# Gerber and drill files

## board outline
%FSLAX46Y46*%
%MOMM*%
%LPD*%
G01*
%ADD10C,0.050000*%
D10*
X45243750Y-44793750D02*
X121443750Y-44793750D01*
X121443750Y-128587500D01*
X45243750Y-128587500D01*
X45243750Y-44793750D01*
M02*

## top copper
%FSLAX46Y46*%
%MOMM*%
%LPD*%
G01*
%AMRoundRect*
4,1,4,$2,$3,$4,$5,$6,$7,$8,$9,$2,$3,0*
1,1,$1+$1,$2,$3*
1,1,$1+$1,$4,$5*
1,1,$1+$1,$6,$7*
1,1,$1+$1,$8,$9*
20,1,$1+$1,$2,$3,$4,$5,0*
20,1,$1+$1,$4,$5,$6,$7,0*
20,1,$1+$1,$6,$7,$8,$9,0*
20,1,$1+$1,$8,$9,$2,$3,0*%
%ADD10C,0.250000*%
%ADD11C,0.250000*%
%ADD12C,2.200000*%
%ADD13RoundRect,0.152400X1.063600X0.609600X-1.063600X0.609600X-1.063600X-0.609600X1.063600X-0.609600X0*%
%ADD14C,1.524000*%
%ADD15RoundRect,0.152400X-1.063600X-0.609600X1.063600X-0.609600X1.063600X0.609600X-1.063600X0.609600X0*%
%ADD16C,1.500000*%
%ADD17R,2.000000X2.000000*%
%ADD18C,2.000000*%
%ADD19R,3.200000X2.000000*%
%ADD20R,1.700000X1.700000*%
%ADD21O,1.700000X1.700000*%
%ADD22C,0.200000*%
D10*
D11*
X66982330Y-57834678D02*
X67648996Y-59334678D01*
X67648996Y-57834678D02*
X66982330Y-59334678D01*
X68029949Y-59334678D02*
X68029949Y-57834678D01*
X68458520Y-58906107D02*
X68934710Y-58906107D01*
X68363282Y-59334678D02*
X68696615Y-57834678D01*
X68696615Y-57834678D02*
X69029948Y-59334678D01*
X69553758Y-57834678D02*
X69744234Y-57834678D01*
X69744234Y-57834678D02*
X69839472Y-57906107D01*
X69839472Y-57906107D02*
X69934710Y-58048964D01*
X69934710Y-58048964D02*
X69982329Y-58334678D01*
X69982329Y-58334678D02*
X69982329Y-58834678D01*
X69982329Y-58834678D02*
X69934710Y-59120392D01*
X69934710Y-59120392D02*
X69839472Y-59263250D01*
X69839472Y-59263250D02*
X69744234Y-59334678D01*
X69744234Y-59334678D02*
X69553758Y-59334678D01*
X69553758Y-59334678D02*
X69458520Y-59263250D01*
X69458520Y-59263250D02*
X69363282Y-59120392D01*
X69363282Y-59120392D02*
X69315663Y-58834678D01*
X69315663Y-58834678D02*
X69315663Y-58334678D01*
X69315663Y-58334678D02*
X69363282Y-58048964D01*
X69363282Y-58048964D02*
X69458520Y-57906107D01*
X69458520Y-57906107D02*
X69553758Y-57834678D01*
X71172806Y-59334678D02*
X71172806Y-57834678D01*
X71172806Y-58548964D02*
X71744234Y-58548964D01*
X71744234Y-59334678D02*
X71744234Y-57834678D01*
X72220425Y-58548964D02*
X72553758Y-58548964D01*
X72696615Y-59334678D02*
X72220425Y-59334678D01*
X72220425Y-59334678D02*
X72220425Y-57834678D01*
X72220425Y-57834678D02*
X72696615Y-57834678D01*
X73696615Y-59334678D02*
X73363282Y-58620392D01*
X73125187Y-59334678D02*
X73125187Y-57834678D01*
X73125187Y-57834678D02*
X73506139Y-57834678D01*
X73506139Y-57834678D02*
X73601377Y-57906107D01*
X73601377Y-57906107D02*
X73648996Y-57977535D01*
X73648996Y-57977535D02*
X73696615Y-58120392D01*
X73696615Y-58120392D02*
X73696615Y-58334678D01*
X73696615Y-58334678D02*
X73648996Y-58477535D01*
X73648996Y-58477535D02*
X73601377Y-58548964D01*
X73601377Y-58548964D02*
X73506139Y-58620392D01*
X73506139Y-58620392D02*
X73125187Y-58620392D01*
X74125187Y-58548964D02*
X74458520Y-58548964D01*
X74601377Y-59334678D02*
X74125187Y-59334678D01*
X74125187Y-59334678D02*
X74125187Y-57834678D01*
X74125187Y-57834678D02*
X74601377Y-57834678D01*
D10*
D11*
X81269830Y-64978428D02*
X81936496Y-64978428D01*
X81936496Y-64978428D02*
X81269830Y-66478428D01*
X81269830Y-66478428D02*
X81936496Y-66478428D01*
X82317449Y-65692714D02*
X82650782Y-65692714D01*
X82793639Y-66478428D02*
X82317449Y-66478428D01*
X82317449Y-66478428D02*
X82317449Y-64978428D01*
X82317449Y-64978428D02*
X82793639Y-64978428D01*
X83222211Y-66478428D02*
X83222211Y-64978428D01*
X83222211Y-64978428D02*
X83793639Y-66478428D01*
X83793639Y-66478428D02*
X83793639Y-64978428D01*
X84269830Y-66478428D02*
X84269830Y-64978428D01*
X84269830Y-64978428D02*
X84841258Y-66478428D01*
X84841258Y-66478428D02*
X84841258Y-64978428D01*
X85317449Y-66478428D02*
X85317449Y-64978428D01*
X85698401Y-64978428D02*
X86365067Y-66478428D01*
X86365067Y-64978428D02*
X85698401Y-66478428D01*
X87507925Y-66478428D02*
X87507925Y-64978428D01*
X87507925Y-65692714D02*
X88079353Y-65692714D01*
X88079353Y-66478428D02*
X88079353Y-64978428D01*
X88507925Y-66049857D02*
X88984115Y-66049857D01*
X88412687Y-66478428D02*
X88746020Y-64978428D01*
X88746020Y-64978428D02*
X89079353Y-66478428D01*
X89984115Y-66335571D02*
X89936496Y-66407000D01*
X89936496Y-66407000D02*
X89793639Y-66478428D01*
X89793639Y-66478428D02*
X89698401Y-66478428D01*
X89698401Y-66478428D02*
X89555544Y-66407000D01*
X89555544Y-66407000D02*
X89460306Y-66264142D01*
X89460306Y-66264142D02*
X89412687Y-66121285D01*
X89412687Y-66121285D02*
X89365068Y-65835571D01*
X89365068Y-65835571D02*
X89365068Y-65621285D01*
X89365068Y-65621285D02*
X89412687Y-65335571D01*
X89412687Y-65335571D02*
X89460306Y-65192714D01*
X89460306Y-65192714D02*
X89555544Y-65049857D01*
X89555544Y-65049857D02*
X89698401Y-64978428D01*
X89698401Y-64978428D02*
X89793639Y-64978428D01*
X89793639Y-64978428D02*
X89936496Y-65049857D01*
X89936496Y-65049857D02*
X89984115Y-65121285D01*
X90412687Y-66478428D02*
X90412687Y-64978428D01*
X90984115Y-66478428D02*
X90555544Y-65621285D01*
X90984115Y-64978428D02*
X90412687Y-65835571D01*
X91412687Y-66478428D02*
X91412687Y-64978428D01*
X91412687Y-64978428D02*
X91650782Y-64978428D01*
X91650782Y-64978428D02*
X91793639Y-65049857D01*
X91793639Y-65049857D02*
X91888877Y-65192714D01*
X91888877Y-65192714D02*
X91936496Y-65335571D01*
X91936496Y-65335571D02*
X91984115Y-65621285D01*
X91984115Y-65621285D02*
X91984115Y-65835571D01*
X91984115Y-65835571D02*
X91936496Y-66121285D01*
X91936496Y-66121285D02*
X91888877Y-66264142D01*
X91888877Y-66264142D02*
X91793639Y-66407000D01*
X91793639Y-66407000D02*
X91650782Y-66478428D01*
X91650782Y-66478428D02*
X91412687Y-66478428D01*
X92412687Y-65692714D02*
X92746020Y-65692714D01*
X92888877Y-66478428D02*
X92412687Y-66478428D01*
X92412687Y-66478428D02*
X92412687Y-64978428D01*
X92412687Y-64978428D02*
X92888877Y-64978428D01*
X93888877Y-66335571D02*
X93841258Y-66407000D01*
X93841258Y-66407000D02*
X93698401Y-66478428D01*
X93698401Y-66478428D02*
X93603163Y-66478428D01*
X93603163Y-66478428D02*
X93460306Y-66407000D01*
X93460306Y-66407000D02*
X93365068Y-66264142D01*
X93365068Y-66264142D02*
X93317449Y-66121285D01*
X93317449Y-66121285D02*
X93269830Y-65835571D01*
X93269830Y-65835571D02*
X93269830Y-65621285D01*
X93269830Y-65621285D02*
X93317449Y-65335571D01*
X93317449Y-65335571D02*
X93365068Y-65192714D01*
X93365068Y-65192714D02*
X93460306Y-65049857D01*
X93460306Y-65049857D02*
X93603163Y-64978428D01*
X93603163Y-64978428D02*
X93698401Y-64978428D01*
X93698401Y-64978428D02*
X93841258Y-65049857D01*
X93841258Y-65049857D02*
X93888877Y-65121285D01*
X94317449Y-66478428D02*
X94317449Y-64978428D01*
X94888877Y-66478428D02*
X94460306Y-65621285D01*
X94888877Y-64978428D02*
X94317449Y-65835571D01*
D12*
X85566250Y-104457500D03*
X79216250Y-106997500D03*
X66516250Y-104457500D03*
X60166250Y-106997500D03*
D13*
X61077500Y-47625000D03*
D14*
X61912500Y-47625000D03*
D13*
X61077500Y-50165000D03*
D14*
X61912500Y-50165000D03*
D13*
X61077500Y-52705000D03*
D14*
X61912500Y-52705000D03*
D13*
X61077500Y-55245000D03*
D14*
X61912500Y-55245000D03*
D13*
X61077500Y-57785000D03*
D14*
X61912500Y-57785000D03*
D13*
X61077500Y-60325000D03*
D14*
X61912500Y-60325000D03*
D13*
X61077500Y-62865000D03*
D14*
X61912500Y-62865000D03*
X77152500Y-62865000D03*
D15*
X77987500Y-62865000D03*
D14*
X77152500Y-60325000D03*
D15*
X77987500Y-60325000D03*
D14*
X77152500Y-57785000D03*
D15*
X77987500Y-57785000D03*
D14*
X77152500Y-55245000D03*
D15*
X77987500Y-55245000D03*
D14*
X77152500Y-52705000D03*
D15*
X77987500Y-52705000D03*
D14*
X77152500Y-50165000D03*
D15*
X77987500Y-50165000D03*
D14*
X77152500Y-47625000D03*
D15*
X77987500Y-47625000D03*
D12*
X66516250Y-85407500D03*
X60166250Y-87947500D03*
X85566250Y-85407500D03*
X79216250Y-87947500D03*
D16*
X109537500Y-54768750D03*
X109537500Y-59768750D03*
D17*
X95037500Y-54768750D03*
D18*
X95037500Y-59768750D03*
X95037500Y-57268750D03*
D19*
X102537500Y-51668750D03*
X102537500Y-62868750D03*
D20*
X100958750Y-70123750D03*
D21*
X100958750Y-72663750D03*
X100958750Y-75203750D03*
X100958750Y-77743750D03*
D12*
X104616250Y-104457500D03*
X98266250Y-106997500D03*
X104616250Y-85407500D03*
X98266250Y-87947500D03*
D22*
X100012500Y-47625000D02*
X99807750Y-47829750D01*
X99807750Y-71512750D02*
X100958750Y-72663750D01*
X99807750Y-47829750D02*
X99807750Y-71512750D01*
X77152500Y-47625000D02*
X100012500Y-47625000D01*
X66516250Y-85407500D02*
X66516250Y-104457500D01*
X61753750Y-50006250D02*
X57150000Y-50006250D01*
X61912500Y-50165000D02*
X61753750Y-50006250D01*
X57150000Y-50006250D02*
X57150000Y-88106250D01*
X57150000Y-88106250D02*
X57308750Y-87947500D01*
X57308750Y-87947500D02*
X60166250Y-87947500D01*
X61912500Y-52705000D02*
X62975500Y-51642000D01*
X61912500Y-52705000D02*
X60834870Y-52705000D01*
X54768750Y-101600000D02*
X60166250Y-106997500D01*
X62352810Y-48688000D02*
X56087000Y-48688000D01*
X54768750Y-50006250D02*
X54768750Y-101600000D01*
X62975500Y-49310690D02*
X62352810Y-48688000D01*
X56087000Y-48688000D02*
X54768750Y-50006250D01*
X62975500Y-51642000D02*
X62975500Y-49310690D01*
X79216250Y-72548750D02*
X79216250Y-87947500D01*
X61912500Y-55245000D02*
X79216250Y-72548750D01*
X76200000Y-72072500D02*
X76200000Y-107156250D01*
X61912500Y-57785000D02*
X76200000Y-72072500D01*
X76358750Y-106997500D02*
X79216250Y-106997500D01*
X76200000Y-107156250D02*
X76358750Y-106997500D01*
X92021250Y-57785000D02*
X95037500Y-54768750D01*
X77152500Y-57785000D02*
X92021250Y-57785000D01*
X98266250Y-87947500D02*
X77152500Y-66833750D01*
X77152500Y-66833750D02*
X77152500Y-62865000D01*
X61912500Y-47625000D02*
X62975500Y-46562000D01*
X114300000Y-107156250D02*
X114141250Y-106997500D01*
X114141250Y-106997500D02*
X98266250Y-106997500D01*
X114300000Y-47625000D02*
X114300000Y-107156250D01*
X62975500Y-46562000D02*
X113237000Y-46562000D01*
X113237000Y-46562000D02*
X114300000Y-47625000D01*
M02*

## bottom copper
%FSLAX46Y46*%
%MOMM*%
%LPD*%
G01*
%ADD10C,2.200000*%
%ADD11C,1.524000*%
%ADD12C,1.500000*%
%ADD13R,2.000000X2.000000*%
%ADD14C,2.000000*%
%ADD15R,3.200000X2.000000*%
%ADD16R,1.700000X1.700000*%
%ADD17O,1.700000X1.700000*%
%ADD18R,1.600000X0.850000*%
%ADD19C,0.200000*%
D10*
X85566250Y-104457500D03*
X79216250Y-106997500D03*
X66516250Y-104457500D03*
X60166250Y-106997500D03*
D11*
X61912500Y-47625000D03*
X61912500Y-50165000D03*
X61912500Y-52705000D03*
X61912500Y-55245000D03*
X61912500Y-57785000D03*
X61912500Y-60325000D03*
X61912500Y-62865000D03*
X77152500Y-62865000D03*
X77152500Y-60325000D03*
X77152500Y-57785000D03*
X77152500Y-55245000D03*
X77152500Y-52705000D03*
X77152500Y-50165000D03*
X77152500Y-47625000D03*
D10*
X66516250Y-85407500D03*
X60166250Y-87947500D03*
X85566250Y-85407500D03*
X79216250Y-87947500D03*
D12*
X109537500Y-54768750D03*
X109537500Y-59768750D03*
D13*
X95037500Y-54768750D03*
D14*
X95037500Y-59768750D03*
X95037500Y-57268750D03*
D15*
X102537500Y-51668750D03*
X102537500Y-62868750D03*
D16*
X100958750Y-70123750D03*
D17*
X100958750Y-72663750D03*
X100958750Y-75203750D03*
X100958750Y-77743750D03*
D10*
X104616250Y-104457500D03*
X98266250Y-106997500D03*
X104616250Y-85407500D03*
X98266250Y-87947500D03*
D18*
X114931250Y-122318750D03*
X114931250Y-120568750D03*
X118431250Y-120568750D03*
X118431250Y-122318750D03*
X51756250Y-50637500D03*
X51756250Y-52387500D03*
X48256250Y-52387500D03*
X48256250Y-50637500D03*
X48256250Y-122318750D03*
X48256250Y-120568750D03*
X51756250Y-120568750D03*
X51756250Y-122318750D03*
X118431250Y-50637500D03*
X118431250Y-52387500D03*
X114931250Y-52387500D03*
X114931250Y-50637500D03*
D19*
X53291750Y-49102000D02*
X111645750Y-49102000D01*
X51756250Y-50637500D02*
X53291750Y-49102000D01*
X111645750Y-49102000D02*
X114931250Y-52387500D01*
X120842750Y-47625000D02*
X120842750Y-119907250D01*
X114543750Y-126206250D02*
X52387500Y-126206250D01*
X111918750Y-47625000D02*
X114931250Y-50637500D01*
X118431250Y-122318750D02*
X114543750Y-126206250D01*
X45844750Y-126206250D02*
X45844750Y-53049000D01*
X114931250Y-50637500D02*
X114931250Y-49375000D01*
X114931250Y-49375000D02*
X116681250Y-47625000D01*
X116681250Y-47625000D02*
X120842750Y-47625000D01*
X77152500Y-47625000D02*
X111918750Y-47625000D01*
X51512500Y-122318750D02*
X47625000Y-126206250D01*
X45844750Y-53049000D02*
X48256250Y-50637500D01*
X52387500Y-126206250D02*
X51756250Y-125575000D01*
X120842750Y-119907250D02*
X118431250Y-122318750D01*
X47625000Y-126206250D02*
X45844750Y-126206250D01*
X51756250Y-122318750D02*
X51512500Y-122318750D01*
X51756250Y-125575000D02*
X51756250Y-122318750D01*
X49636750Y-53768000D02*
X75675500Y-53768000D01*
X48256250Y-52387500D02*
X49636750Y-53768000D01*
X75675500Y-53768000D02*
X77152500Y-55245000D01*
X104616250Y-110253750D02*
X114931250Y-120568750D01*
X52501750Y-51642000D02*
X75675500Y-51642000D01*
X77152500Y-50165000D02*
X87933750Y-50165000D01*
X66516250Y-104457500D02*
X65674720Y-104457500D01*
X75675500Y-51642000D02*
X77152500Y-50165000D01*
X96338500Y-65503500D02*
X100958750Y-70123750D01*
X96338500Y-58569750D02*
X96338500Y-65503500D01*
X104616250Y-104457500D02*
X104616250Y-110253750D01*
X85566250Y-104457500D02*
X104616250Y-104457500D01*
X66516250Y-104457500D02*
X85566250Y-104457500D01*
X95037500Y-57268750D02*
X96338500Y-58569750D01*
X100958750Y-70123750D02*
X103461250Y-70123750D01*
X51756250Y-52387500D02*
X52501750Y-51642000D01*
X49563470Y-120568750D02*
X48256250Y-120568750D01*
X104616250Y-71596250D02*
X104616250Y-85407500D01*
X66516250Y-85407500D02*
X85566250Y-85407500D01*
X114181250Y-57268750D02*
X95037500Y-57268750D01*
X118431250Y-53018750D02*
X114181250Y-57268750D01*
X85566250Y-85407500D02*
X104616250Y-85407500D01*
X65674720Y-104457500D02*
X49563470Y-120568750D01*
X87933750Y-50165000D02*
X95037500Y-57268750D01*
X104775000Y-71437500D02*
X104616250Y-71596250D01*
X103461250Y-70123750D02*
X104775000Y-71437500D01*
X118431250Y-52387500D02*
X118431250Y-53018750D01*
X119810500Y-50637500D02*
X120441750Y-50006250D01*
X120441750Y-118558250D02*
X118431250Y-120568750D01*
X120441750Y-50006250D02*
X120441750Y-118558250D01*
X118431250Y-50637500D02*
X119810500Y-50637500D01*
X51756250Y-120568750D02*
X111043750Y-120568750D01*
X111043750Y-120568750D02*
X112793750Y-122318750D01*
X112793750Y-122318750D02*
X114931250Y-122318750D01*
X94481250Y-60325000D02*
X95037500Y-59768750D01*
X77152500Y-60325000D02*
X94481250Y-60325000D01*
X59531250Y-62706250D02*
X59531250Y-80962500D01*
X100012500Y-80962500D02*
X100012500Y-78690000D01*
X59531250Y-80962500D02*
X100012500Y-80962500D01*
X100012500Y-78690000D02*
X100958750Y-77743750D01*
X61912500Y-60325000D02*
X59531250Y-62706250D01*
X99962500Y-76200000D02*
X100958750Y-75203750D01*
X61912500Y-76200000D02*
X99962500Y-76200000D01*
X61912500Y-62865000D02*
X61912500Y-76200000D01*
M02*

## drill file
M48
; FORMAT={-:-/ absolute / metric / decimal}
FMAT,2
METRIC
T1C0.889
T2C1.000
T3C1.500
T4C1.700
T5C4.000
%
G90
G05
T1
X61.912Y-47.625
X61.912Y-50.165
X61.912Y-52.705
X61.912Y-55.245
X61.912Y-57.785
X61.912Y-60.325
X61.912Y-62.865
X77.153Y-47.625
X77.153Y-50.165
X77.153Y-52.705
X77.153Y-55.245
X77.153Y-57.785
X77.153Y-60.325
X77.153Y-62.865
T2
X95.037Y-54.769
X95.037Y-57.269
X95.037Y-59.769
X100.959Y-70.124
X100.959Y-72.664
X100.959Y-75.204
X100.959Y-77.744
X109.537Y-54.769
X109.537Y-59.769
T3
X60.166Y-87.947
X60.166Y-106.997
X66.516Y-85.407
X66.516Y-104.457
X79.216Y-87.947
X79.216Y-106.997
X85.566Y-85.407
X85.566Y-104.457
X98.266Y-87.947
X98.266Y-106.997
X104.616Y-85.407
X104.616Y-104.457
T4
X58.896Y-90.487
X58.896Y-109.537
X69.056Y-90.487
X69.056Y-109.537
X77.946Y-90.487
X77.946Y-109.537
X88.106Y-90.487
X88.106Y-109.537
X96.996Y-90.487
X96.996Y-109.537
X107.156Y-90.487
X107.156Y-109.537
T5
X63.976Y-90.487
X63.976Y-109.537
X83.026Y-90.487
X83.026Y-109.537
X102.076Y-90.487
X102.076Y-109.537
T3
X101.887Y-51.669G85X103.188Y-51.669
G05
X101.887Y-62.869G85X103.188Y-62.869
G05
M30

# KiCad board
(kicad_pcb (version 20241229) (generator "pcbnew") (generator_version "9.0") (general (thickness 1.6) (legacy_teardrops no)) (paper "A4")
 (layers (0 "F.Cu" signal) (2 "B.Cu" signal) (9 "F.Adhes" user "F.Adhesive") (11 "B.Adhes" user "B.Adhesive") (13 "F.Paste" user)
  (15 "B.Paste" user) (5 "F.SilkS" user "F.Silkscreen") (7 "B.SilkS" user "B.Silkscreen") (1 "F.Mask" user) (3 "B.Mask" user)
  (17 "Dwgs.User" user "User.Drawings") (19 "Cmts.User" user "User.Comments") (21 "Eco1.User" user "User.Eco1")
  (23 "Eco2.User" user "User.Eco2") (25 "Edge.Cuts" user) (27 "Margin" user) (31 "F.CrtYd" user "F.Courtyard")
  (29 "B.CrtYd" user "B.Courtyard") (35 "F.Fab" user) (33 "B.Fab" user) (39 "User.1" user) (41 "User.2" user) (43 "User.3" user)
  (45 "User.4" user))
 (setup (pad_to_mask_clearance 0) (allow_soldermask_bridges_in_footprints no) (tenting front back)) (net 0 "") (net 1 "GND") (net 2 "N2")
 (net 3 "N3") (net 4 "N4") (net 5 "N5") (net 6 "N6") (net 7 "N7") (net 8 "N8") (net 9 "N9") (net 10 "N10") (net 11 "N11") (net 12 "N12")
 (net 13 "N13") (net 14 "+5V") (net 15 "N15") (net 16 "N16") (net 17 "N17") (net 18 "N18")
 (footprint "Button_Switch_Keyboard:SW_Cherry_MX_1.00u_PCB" (layer "F.Cu") (at 85.56625 104.4575)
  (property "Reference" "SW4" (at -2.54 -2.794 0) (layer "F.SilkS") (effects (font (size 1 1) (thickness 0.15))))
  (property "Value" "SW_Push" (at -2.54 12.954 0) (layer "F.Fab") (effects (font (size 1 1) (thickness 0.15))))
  (pad "" np_thru_hole circle (at -7.62 5.08) (size 1.7 1.7) (drill 1.7) (layers "*.Cu" "*.Mask"))
  (pad "" np_thru_hole circle (at -2.54 5.08) (size 4 4) (drill 4) (layers "*.Cu" "*.Mask"))
  (pad "" np_thru_hole circle (at 2.54 5.08) (size 1.7 1.7) (drill 1.7) (layers "*.Cu" "*.Mask"))
  (pad "1" thru_hole circle (at 0 0) (size 2.2 2.2) (drill 1.5) (layers "*.Cu" "*.Mask") (remove_unused_layers no) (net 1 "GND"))
  (pad "2" thru_hole circle (at -6.35 2.54) (size 2.2 2.2) (drill 1.5) (layers "*.Cu" "*.Mask") (remove_unused_layers no) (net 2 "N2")))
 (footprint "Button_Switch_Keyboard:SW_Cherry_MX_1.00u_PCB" (layer "F.Cu") (at 66.51625 104.4575)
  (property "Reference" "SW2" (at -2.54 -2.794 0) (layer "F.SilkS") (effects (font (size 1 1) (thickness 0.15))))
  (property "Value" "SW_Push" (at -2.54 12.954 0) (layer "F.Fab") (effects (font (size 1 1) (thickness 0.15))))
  (pad "" np_thru_hole circle (at -7.62 5.08) (size 1.7 1.7) (drill 1.7) (layers "*.Cu" "*.Mask"))
  (pad "" np_thru_hole circle (at -2.54 5.08) (size 4 4) (drill 4) (layers "*.Cu" "*.Mask"))
  (pad "" np_thru_hole circle (at 2.54 5.08) (size 1.7 1.7) (drill 1.7) (layers "*.Cu" "*.Mask"))
  (pad "1" thru_hole circle (at 0 0) (size 2.2 2.2) (drill 1.5) (layers "*.Cu" "*.Mask") (remove_unused_layers no) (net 1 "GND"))
  (pad "2" thru_hole circle (at -6.35 2.54) (size 2.2 2.2) (drill 1.5) (layers "*.Cu" "*.Mask") (remove_unused_layers no) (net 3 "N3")))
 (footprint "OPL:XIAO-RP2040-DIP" (layer "F.Cu") (at 69.5325 55.245)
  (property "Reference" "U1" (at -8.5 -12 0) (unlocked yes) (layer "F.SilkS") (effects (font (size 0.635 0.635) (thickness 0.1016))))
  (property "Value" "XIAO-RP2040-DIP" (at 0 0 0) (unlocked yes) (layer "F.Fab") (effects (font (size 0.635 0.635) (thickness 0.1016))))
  (pad "1" smd roundrect (at -8.455 -7.62 180) (size 2.432 1.524) (layers "F.Cu" "F.Mask") (roundrect_rratio 0.1) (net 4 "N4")
   (thermal_bridge_angle 45))
  (pad "1" thru_hole circle (at -7.62 -7.62 180) (size 1.524 1.524) (drill 0.889) (layers "*.Cu" "*.Mask") (remove_unused_layers no)
   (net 4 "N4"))
  (pad "2" smd roundrect (at -8.455 -5.08 180) (size 2.432 1.524) (layers "F.Cu" "F.Mask") (roundrect_rratio 0.1) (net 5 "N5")
   (thermal_bridge_angle 45))
  (pad "2" thru_hole circle (at -7.62 -5.08 180) (size 1.524 1.524) (drill 0.889) (layers "*.Cu" "*.Mask") (remove_unused_layers no)
   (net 5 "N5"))
  (pad "3" smd roundrect (at -8.455 -2.54 180) (size 2.432 1.524) (layers "F.Cu" "F.Mask") (roundrect_rratio 0.1) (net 3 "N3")
   (thermal_bridge_angle 45))
  (pad "3" thru_hole circle (at -7.62 -2.54 180) (size 1.524 1.524) (drill 0.889) (layers "*.Cu" "*.Mask") (remove_unused_layers no)
   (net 3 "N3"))
  (pad "4" smd roundrect (at -8.455 0 180) (size 2.432 1.524) (layers "F.Cu" "F.Mask") (roundrect_rratio 0.1) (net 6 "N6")
   (thermal_bridge_angle 45))
  (pad "4" thru_hole circle (at -7.62 0 180) (size 1.524 1.524) (drill 0.889) (layers "*.Cu" "*.Mask") (remove_unused_layers no)
   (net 6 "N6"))
  (pad "5" smd roundrect (at -8.455 2.54 180) (size 2.432 1.524) (layers "F.Cu" "F.Mask") (roundrect_rratio 0.1) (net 2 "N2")
   (thermal_bridge_angle 45))
  (pad "5" thru_hole circle (at -7.62 2.54 180) (size 1.524 1.524) (drill 0.889) (layers "*.Cu" "*.Mask") (remove_unused_layers no)
   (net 2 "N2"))
  (pad "6" smd roundrect (at -8.455 5.08 180) (size 2.432 1.524) (layers "F.Cu" "F.Mask") (roundrect_rratio 0.1) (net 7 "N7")
   (thermal_bridge_angle 45))
  (pad "6" thru_hole circle (at -7.62 5.08 180) (size 1.524 1.524) (drill 0.889) (layers "*.Cu" "*.Mask") (remove_unused_layers no)
   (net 7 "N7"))
  (pad "7" smd roundrect (at -8.455 7.62 180) (size 2.432 1.524) (layers "F.Cu" "F.Mask") (roundrect_rratio 0.1) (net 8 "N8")
   (thermal_bridge_angle 45))
  (pad "7" thru_hole circle (at -7.62 7.62 180) (size 1.524 1.524) (drill 0.889) (layers "*.Cu" "*.Mask") (remove_unused_layers no)
   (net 8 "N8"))
  (pad "8" thru_hole circle (at 7.62 7.62) (size 1.524 1.524) (drill 0.889) (layers "*.Cu" "*.Mask") (remove_unused_layers no) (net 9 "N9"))
  (pad "8" smd roundrect (at 8.455 7.62) (size 2.432 1.524) (layers "F.Cu" "F.Mask") (roundrect_rratio 0.1) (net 9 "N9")
   (thermal_bridge_angle 45))
  (pad "9" thru_hole circle (at 7.62 5.08) (size 1.524 1.524) (drill 0.889) (layers "*.Cu" "*.Mask") (remove_unused_layers no)
   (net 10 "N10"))
  (pad "9" smd roundrect (at 8.455 5.08) (size 2.432 1.524) (layers "F.Cu" "F.Mask") (roundrect_rratio 0.1) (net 10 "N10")
   (thermal_bridge_angle 45))
  (pad "10" thru_hole circle (at 7.62 2.54) (size 1.524 1.524) (drill 0.889) (layers "*.Cu" "*.Mask") (remove_unused_layers no)
   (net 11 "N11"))
  (pad "10" smd roundrect (at 8.455 2.54) (size 2.432 1.524) (layers "F.Cu" "F.Mask") (roundrect_rratio 0.1) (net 11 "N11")
   (thermal_bridge_angle 45))
  (pad "11" thru_hole circle (at 7.62 0) (size 1.524 1.524) (drill 0.889) (layers "*.Cu" "*.Mask") (remove_unused_layers no) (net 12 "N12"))
  (pad "11" smd roundrect (at 8.455 0) (size 2.432 1.524) (layers "F.Cu" "F.Mask") (roundrect_rratio 0.1) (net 12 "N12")
   (thermal_bridge_angle 45))
  (pad "12" thru_hole circle (at 7.62 -2.54) (size 1.524 1.524) (drill 0.889) (layers "*.Cu" "*.Mask") (remove_unused_layers no)
   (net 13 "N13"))
  (pad "12" smd roundrect (at 8.455 -2.54) (size 2.432 1.524) (layers "F.Cu" "F.Mask") (roundrect_rratio 0.1) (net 13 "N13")
   (thermal_bridge_angle 45))
  (pad "13" thru_hole circle (at 7.62 -5.08) (size 1.524 1.524) (drill 0.889) (layers "*.Cu" "*.Mask") (remove_unused_layers no)
   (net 1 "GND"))
  (pad "13" smd roundrect (at 8.455 -5.08) (size 2.432 1.524) (layers "F.Cu" "F.Mask") (roundrect_rratio 0.1) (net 1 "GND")
   (thermal_bridge_angle 45))
  (pad "14" thru_hole circle (at 7.62 -7.62) (size 1.524 1.524) (drill 0.889) (layers "*.Cu" "*.Mask") (remove_unused_layers no)
   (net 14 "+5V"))
  (pad "14" smd roundrect (at 8.455 -7.62) (size 2.432 1.524) (layers "F.Cu" "F.Mask") (roundrect_rratio 0.1) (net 14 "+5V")
   (thermal_bridge_angle 45)))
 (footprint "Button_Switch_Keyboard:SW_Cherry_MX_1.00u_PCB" (layer "F.Cu") (at 66.51625 85.4075)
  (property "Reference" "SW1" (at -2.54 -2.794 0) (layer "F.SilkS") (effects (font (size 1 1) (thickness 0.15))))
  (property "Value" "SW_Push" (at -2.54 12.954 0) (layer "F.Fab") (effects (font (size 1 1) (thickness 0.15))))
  (pad "" np_thru_hole circle (at -7.62 5.08) (size 1.7 1.7) (drill 1.7) (layers "*.Cu" "*.Mask"))
  (pad "" np_thru_hole circle (at -2.54 5.08) (size 4 4) (drill 4) (layers "*.Cu" "*.Mask"))
  (pad "" np_thru_hole circle (at 2.54 5.08) (size 1.7 1.7) (drill 1.7) (layers "*.Cu" "*.Mask"))
  (pad "1" thru_hole circle (at 0 0) (size 2.2 2.2) (drill 1.5) (layers "*.Cu" "*.Mask") (remove_unused_layers no) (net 1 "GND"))
  (pad "2" thru_hole circle (at -6.35 2.54) (size 2.2 2.2) (drill 1.5) (layers "*.Cu" "*.Mask") (remove_unused_layers no) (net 5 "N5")))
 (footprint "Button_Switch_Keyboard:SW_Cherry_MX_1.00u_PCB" (layer "F.Cu") (at 85.56625 85.4075)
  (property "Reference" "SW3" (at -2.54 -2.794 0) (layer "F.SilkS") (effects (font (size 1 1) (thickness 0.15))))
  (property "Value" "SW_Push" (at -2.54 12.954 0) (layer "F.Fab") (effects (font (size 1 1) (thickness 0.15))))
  (pad "" np_thru_hole circle (at -7.62 5.08) (size 1.7 1.7) (drill 1.7) (layers "*.Cu" "*.Mask"))
  (pad "" np_thru_hole circle (at -2.54 5.08) (size 4 4) (drill 4) (layers "*.Cu" "*.Mask"))
  (pad "" np_thru_hole circle (at 2.54 5.08) (size 1.7 1.7) (drill 1.7) (layers "*.Cu" "*.Mask"))
  (pad "1" thru_hole circle (at 0 0) (size 2.2 2.2) (drill 1.5) (layers "*.Cu" "*.Mask") (remove_unused_layers no) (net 1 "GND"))
  (pad "2" thru_hole circle (at -6.35 2.54) (size 2.2 2.2) (drill 1.5) (layers "*.Cu" "*.Mask") (remove_unused_layers no) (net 6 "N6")))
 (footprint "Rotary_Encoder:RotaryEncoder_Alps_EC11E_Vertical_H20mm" (layer "F.Cu") (at 95.0375 54.76875)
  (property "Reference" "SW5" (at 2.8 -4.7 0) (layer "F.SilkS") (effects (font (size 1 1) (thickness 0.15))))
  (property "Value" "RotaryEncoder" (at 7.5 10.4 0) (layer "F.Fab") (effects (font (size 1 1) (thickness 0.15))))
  (pad "" thru_hole circle (at 14.5 0) (size 1.5 1.5) (drill 1) (layers "*.Cu" "*.Mask") (remove_unused_layers no))
  (pad "" thru_hole circle (at 14.5 5) (size 1.5 1.5) (drill 1) (layers "*.Cu" "*.Mask") (remove_unused_layers no))
  (pad "A" thru_hole rect (at 0 0) (size 2 2) (drill 1) (layers "*.Cu" "*.Mask") (remove_unused_layers no) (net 11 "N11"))
  (pad "B" thru_hole circle (at 0 5) (size 2 2) (drill 1) (layers "*.Cu" "*.Mask") (remove_unused_layers no) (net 10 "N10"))
  (pad "C" thru_hole circle (at 0 2.5) (size 2 2) (drill 1) (layers "*.Cu" "*.Mask") (remove_unused_layers no) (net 1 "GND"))
  (pad "MP" thru_hole rect (at 7.5 -3.1) (size 3.2 2) (drill oval 2.8 1.5) (layers "*.Cu" "*.Mask") (remove_unused_layers no))
  (pad "MP" thru_hole rect (at 7.5 8.1) (size 3.2 2) (drill oval 2.8 1.5) (layers "*.Cu" "*.Mask") (remove_unused_layers no)))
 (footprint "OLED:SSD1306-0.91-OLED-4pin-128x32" (layer "F.Cu") (at 64.45875 67.93375)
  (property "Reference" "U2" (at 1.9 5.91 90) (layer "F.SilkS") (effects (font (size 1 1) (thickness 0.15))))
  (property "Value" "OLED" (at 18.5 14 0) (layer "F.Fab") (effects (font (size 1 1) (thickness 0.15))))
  (pad "1" thru_hole rect (at 36.5 2.19) (size 1.7 1.7) (drill 1) (layers "*.Cu" "*.Mask") (remove_unused_layers no) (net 1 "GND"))
  (pad "2" thru_hole oval (at 36.5 4.73) (size 1.7 1.7) (drill 1) (layers "*.Cu" "*.Mask") (remove_unused_layers no) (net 14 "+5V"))
  (pad "3" thru_hole oval (at 36.5 7.27) (size 1.7 1.7) (drill 1) (layers "*.Cu" "*.Mask") (remove_unused_layers no) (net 8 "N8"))
  (pad "4" thru_hole oval (at 36.5 9.81) (size 1.7 1.7) (drill 1) (layers "*.Cu" "*.Mask") (remove_unused_layers no) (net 7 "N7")))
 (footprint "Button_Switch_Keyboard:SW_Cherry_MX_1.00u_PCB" (layer "F.Cu") (at 104.61625 104.4575)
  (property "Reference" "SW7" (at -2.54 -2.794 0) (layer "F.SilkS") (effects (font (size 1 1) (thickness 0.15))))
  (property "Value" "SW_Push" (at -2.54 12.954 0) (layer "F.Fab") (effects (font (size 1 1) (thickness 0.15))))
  (pad "" np_thru_hole circle (at -7.62 5.08) (size 1.7 1.7) (drill 1.7) (layers "*.Cu" "*.Mask"))
  (pad "" np_thru_hole circle (at -2.54 5.08) (size 4 4) (drill 4) (layers "*.Cu" "*.Mask"))
  (pad "" np_thru_hole circle (at 2.54 5.08) (size 1.7 1.7) (drill 1.7) (layers "*.Cu" "*.Mask"))
  (pad "1" thru_hole circle (at 0 0) (size 2.2 2.2) (drill 1.5) (layers "*.Cu" "*.Mask") (remove_unused_layers no) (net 1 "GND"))
  (pad "2" thru_hole circle (at -6.35 2.54) (size 2.2 2.2) (drill 1.5) (layers "*.Cu" "*.Mask") (remove_unused_layers no) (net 4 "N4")))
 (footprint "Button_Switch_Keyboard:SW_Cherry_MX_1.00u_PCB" (layer "F.Cu") (at 104.61625 85.4075)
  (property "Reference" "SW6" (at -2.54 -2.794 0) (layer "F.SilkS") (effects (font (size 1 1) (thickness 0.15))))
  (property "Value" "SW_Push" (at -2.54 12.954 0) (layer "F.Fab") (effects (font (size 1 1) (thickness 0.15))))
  (pad "" np_thru_hole circle (at -7.62 5.08) (size 1.7 1.7) (drill 1.7) (layers "*.Cu" "*.Mask"))
  (pad "" np_thru_hole circle (at -2.54 5.08) (size 4 4) (drill 4) (layers "*.Cu" "*.Mask"))
  (pad "" np_thru_hole circle (at 2.54 5.08) (size 1.7 1.7) (drill 1.7) (layers "*.Cu" "*.Mask"))
  (pad "1" thru_hole circle (at 0 0) (size 2.2 2.2) (drill 1.5) (layers "*.Cu" "*.Mask") (remove_unused_layers no) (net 1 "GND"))
  (pad "2" thru_hole circle (at -6.35 2.54) (size 2.2 2.2) (drill 1.5) (layers "*.Cu" "*.Mask") (remove_unused_layers no) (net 9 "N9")))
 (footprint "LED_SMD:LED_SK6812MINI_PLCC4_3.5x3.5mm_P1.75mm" (layer "B.Cu") (at 116.68125 121.44375)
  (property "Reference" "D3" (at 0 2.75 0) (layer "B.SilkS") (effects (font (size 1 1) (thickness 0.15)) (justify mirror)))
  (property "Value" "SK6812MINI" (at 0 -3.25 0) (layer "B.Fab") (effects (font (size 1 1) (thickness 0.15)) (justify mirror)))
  (pad "1" smd rect (at -1.75 0.875) (size 1.6 0.85) (layers "B.Cu" "B.Mask" "B.Paste") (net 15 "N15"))
  (pad "2" smd rect (at -1.75 -0.875) (size 1.6 0.85) (layers "B.Cu" "B.Mask" "B.Paste") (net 1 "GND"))
  (pad "3" smd rect (at 1.75 -0.875) (size 1.6 0.85) (layers "B.Cu" "B.Mask" "B.Paste") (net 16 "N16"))
  (pad "4" smd rect (at 1.75 0.875) (size 1.6 0.85) (layers "B.Cu" "B.Mask" "B.Paste") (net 14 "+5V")))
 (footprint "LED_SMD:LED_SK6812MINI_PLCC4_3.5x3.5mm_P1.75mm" (layer "B.Cu") (at 50.00625 51.5125 180)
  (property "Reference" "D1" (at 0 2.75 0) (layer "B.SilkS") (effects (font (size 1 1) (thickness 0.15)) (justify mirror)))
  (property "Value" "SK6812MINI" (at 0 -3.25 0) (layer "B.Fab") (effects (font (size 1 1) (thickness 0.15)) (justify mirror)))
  (pad "1" smd rect (at -1.75 0.875 180) (size 1.6 0.85) (layers "B.Cu" "B.Mask" "B.Paste") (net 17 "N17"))
  (pad "2" smd rect (at -1.75 -0.875 180) (size 1.6 0.85) (layers "B.Cu" "B.Mask" "B.Paste") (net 1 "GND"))
  (pad "3" smd rect (at 1.75 -0.875 180) (size 1.6 0.85) (layers "B.Cu" "B.Mask" "B.Paste") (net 12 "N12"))
  (pad "4" smd rect (at 1.75 0.875 180) (size 1.6 0.85) (layers "B.Cu" "B.Mask" "B.Paste") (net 14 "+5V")))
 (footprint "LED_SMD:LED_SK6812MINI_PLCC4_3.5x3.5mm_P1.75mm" (layer "B.Cu") (at 50.00625 121.44375)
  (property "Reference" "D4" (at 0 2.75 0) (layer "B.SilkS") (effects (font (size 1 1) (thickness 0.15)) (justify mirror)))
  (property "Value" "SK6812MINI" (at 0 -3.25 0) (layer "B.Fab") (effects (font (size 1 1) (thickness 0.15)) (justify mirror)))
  (pad "1" smd rect (at -1.75 0.875) (size 1.6 0.85) (layers "B.Cu" "B.Mask" "B.Paste") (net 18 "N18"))
  (pad "2" smd rect (at -1.75 -0.875) (size 1.6 0.85) (layers "B.Cu" "B.Mask" "B.Paste") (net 1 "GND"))
  (pad "3" smd rect (at 1.75 -0.875) (size 1.6 0.85) (layers "B.Cu" "B.Mask" "B.Paste") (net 15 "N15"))
  (pad "4" smd rect (at 1.75 0.875) (size 1.6 0.85) (layers "B.Cu" "B.Mask" "B.Paste") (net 14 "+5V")))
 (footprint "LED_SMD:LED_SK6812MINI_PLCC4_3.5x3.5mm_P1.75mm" (layer "B.Cu") (at 116.68125 51.5125 180)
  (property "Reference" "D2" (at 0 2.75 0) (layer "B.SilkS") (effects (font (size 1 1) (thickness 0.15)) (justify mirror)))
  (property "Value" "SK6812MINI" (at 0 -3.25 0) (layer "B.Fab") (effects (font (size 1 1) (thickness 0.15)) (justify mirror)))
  (pad "1" smd rect (at -1.75 0.875 180) (size 1.6 0.85) (layers "B.Cu" "B.Mask" "B.Paste") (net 16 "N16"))
  (pad "2" smd rect (at -1.75 -0.875 180) (size 1.6 0.85) (layers "B.Cu" "B.Mask" "B.Paste") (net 1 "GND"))
  (pad "3" smd rect (at 1.75 -0.875 180) (size 1.6 0.85) (layers "B.Cu" "B.Mask" "B.Paste") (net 17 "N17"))
  (pad "4" smd rect (at 1.75 0.875 180) (size 1.6 0.85) (layers "B.Cu" "B.Mask" "B.Paste") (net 14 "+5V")))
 (gr_rect (start 45.24375 44.79375) (end 121.44375 128.5875) (stroke (width 0.05) (type default)) (fill no) (layer "Edge.Cuts"))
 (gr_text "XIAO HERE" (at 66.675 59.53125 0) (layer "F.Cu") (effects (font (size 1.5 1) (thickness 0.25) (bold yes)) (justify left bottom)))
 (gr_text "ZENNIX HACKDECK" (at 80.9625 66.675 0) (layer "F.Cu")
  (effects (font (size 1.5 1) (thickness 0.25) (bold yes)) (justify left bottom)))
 (segment (start 53.29175 49.102) (end 111.64575 49.102) (width 0.2) (layer "B.Cu") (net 17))
 (segment (start 51.75625 50.6375) (end 53.29175 49.102) (width 0.2) (layer "B.Cu") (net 17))
 (segment (start 111.64575 49.102) (end 114.93125 52.3875) (width 0.2) (layer "B.Cu") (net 17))
 (segment (start 100.0125 47.625) (end 99.80775 47.82975) (width 0.2) (layer "F.Cu") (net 14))
 (segment (start 99.80775 71.51275) (end 100.95875 72.66375) (width 0.2) (layer "F.Cu") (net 14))
 (segment (start 99.80775 47.82975) (end 99.80775 71.51275) (width 0.2) (layer "F.Cu") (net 14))
 (segment (start 77.1525 47.625) (end 100.0125 47.625) (width 0.2) (layer "F.Cu") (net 14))
 (segment (start 120.84275 47.625) (end 120.84275 119.90725) (width 0.2) (layer "B.Cu") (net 14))
 (segment (start 114.54375 126.20625) (end 52.3875 126.20625) (width 0.2) (layer "B.Cu") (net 14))
 (segment (start 111.91875 47.625) (end 114.93125 50.6375) (width 0.2) (layer "B.Cu") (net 14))
 (segment (start 118.43125 122.31875) (end 114.54375 126.20625) (width 0.2) (layer "B.Cu") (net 14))
 (segment (start 45.84475 126.20625) (end 45.84475 53.049) (width 0.2) (layer "B.Cu") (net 14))
 (segment (start 114.93125 50.6375) (end 114.93125 49.375) (width 0.2) (layer "B.Cu") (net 14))
 (segment (start 114.93125 49.375) (end 116.68125 47.625) (width 0.2) (layer "B.Cu") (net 14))
 (segment (start 116.68125 47.625) (end 120.84275 47.625) (width 0.2) (layer "B.Cu") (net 14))
 (segment (start 77.1525 47.625) (end 111.91875 47.625) (width 0.2) (layer "B.Cu") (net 14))
 (segment (start 51.5125 122.31875) (end 47.625 126.20625) (width 0.2) (layer "B.Cu") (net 14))
 (segment (start 45.84475 53.049) (end 48.25625 50.6375) (width 0.2) (layer "B.Cu") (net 14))
 (segment (start 52.3875 126.20625) (end 51.75625 125.575) (width 0.2) (layer "B.Cu") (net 14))
 (segment (start 120.84275 119.90725) (end 118.43125 122.31875) (width 0.2) (layer "B.Cu") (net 14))
 (segment (start 47.625 126.20625) (end 45.84475 126.20625) (width 0.2) (layer "B.Cu") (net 14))
 (segment (start 51.75625 122.31875) (end 51.5125 122.31875) (width 0.2) (layer "B.Cu") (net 14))
 (segment (start 51.75625 125.575) (end 51.75625 122.31875) (width 0.2) (layer "B.Cu") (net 14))
 (segment (start 49.63675 53.768) (end 75.6755 53.768) (width 0.2) (layer "B.Cu") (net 12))
 (segment (start 48.25625 52.3875) (end 49.63675 53.768) (width 0.2) (layer "B.Cu") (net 12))
 (segment (start 75.6755 53.768) (end 77.1525 55.245) (width 0.2) (layer "B.Cu") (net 12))
 (segment (start 66.51625 85.4075) (end 66.51625 104.4575) (width 0.2) (layer "F.Cu") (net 1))
 (segment (start 104.61625 110.25375) (end 114.93125 120.56875) (width 0.2) (layer "B.Cu") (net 1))
 (segment (start 52.50175 51.642) (end 75.6755 51.642) (width 0.2) (layer "B.Cu") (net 1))
 (segment (start 77.1525 50.165) (end 87.93375 50.165) (width 0.2) (layer "B.Cu") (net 1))
 (segment (start 66.51625 104.4575) (end 65.67472 104.4575) (width 0.2) (layer "B.Cu") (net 1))
 (segment (start 75.6755 51.642) (end 77.1525 50.165) (width 0.2) (layer "B.Cu") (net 1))
 (segment (start 96.3385 65.5035) (end 100.95875 70.12375) (width 0.2) (layer "B.Cu") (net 1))
 (segment (start 96.3385 58.56975) (end 96.3385 65.5035) (width 0.2) (layer "B.Cu") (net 1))
 (segment (start 104.61625 104.4575) (end 104.61625 110.25375) (width 0.2) (layer "B.Cu") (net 1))
 (segment (start 85.56625 104.4575) (end 104.61625 104.4575) (width 0.2) (layer "B.Cu") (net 1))
 (segment (start 66.51625 104.4575) (end 85.56625 104.4575) (width 0.2) (layer "B.Cu") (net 1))
 (segment (start 95.0375 57.26875) (end 96.3385 58.56975) (width 0.2) (layer "B.Cu") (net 1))
 (segment (start 100.95875 70.12375) (end 103.46125 70.12375) (width 0.2) (layer "B.Cu") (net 1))
 (segment (start 51.75625 52.3875) (end 52.50175 51.642) (width 0.2) (layer "B.Cu") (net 1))
 (segment (start 49.56347 120.56875) (end 48.25625 120.56875) (width 0.2) (layer "B.Cu") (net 1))
 (segment (start 104.61625 71.59625) (end 104.61625 85.4075) (width 0.2) (layer "B.Cu") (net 1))
 (segment (start 66.51625 85.4075) (end 85.56625 85.4075) (width 0.2) (layer "B.Cu") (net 1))
 (segment (start 114.18125 57.26875) (end 95.0375 57.26875) (width 0.2) (layer "B.Cu") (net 1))
 (segment (start 118.43125 53.01875) (end 114.18125 57.26875) (width 0.2) (layer "B.Cu") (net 1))
 (segment (start 85.56625 85.4075) (end 104.61625 85.4075) (width 0.2) (layer "B.Cu") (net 1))
 (segment (start 65.67472 104.4575) (end 49.56347 120.56875) (width 0.2) (layer "B.Cu") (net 1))
 (segment (start 87.93375 50.165) (end 95.0375 57.26875) (width 0.2) (layer "B.Cu") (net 1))
 (segment (start 104.775 71.4375) (end 104.61625 71.59625) (width 0.2) (layer "B.Cu") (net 1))
 (segment (start 103.46125 70.12375) (end 104.775 71.4375) (width 0.2) (layer "B.Cu") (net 1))
 (segment (start 118.43125 52.3875) (end 118.43125 53.01875) (width 0.2) (layer "B.Cu") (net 1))
 (segment (start 119.8105 50.6375) (end 120.44175 50.00625) (width 0.2) (layer "B.Cu") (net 16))
 (segment (start 120.44175 118.55825) (end 118.43125 120.56875) (width 0.2) (layer "B.Cu") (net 16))
 (segment (start 120.44175 50.00625) (end 120.44175 118.55825) (width 0.2) (layer "B.Cu") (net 16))
 (segment (start 118.43125 50.6375) (end 119.8105 50.6375) (width 0.2) (layer "B.Cu") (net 16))
 (segment (start 51.75625 120.56875) (end 111.04375 120.56875) (width 0.2) (layer "B.Cu") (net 15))
 (segment (start 111.04375 120.56875) (end 112.79375 122.31875) (width 0.2) (layer "B.Cu") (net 15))
 (segment (start 112.79375 122.31875) (end 114.93125 122.31875) (width 0.2) (layer "B.Cu") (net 15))
 (segment (start 61.75375 50.00625) (end 57.15 50.00625) (width 0.2) (layer "F.Cu") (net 5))
 (segment (start 61.9125 50.165) (end 61.75375 50.00625) (width 0.2) (layer "F.Cu") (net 5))
 (segment (start 57.15 50.00625) (end 57.15 88.10625) (width 0.2) (layer "F.Cu") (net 5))
 (segment (start 57.15 88.10625) (end 57.30875 87.9475) (width 0.2) (layer "F.Cu") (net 5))
 (segment (start 57.30875 87.9475) (end 60.16625 87.9475) (width 0.2) (layer "F.Cu") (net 5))
 (segment (start 61.9125 52.705) (end 62.9755 51.642) (width 0.2) (layer "F.Cu") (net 3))
 (segment (start 61.9125 52.705) (end 60.83487 52.705) (width 0.2) (layer "F.Cu") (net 3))
 (segment (start 54.76875 101.6) (end 60.16625 106.9975) (width 0.2) (layer "F.Cu") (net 3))
 (segment (start 62.35281 48.688) (end 56.087 48.688) (width 0.2) (layer "F.Cu") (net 3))
 (segment (start 54.76875 50.00625) (end 54.76875 101.6) (width 0.2) (layer "F.Cu") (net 3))
 (segment (start 62.9755 49.31069) (end 62.35281 48.688) (width 0.2) (layer "F.Cu") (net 3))
 (segment (start 56.087 48.688) (end 54.76875 50.00625) (width 0.2) (layer "F.Cu") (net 3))
 (segment (start 62.9755 51.642) (end 62.9755 49.31069) (width 0.2) (layer "F.Cu") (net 3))
 (segment (start 79.21625 72.54875) (end 79.21625 87.9475) (width 0.2) (layer "F.Cu") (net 6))
 (segment (start 61.9125 55.245) (end 79.21625 72.54875) (width 0.2) (layer "F.Cu") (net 6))
 (segment (start 76.2 72.0725) (end 76.2 107.15625) (width 0.2) (layer "F.Cu") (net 2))
 (segment (start 61.9125 57.785) (end 76.2 72.0725) (width 0.2) (layer "F.Cu") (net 2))
 (segment (start 76.35875 106.9975) (end 79.21625 106.9975) (width 0.2) (layer "F.Cu") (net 2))
 (segment (start 76.2 107.15625) (end 76.35875 106.9975) (width 0.2) (layer "F.Cu") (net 2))
 (segment (start 94.48125 60.325) (end 95.0375 59.76875) (width 0.2) (layer "B.Cu") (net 10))
 (segment (start 77.1525 60.325) (end 94.48125 60.325) (width 0.2) (layer "B.Cu") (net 10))
 (segment (start 92.02125 57.785) (end 95.0375 54.76875) (width 0.2) (layer "F.Cu") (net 11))
 (segment (start 77.1525 57.785) (end 92.02125 57.785) (width 0.2) (layer "F.Cu") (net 11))
 (segment (start 98.26625 87.9475) (end 77.1525 66.83375) (width 0.2) (layer "F.Cu") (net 9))
 (segment (start 77.1525 66.83375) (end 77.1525 62.865) (width 0.2) (layer "F.Cu") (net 9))
 (segment (start 61.9125 47.625) (end 62.9755 46.562) (width 0.2) (layer "F.Cu") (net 4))
 (segment (start 114.3 107.15625) (end 114.14125 106.9975) (width 0.2) (layer "F.Cu") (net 4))
 (segment (start 114.14125 106.9975) (end 98.26625 106.9975) (width 0.2) (layer "F.Cu") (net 4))
 (segment (start 114.3 47.625) (end 114.3 107.15625) (width 0.2) (layer "F.Cu") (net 4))
 (segment (start 62.9755 46.562) (end 113.237 46.562) (width 0.2) (layer "F.Cu") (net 4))
 (segment (start 113.237 46.562) (end 114.3 47.625) (width 0.2) (layer "F.Cu") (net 4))
 (segment (start 59.53125 62.70625) (end 59.53125 80.9625) (width 0.2) (layer "B.Cu") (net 7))
 (segment (start 100.0125 80.9625) (end 100.0125 78.69) (width 0.2) (layer "B.Cu") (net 7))
 (segment (start 59.53125 80.9625) (end 100.0125 80.9625) (width 0.2) (layer "B.Cu") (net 7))
 (segment (start 100.0125 78.69) (end 100.95875 77.74375) (width 0.2) (layer "B.Cu") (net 7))
 (segment (start 61.9125 60.325) (end 59.53125 62.70625) (width 0.2) (layer "B.Cu") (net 7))
 (segment (start 99.9625 76.2) (end 100.95875 75.20375) (width 0.2) (layer "B.Cu") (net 8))
 (segment (start 61.9125 76.2) (end 99.9625 76.2) (width 0.2) (layer "B.Cu") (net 8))
 (segment (start 61.9125 62.865) (end 61.9125 76.2) (width 0.2) (layer "B.Cu") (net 8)))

